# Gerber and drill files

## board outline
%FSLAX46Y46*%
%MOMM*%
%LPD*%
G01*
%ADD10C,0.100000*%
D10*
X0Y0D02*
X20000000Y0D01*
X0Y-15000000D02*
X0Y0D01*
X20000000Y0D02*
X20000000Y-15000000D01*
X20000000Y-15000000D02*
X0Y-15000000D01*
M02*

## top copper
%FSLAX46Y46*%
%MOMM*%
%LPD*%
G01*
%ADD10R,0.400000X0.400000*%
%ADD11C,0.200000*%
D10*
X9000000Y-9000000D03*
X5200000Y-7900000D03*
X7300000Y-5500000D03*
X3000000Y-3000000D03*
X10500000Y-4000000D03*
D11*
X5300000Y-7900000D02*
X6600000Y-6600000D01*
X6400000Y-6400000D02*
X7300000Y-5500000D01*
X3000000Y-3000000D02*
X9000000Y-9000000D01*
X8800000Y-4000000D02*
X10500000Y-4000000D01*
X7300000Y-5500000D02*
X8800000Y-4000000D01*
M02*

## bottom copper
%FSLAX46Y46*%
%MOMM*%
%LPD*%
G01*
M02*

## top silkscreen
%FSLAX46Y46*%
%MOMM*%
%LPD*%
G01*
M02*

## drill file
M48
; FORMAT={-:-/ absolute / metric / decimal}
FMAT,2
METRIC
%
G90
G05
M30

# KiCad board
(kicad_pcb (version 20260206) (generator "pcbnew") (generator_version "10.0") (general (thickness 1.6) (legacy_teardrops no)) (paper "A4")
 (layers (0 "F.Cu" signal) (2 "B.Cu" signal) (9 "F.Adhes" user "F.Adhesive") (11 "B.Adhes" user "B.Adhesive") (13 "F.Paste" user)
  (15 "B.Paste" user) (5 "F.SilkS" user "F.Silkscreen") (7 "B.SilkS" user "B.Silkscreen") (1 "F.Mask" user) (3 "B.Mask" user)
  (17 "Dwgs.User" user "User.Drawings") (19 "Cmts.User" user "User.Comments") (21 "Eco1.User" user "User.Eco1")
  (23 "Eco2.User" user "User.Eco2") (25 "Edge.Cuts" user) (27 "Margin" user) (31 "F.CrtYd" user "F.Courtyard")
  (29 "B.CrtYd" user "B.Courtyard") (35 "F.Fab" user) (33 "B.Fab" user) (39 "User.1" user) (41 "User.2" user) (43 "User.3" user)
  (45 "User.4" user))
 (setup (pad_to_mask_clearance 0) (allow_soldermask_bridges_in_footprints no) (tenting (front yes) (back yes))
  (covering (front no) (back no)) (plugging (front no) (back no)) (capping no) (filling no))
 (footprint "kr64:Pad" (layer "F.Cu") (at 9 9)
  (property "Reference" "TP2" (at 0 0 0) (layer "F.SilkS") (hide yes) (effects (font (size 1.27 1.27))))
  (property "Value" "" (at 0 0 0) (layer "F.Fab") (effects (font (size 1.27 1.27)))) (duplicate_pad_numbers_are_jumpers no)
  (pad "1" smd rect (at 0 0) (size 0.4 0.4) (layers "F.Cu" "F.Mask" "F.Paste") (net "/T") (thermal_bridge_angle 45)))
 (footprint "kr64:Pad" (layer "F.Cu") (at 5.2 7.9)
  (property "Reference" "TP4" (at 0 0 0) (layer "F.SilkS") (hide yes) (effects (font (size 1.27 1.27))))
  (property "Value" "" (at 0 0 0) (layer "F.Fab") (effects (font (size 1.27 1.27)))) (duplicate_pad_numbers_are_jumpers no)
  (pad "1" smd rect (at 0 0) (size 0.4 0.4) (layers "F.Cu" "F.Mask" "F.Paste") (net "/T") (thermal_bridge_angle 45)))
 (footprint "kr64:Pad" (layer "F.Cu") (at 7.3 5.5)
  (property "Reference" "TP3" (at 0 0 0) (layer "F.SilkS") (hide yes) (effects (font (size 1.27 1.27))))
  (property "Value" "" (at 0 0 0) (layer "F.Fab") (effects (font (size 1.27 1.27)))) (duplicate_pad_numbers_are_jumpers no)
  (pad "1" smd rect (at 0 0) (size 0.4 0.4) (layers "F.Cu" "F.Mask" "F.Paste") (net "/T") (thermal_bridge_angle 45)))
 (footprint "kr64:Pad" (layer "F.Cu") (at 3 3)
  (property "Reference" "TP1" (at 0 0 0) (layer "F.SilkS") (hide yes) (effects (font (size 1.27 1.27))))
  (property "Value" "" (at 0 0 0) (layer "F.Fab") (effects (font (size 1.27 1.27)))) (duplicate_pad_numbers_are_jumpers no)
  (pad "1" smd rect (at 0 0) (size 0.4 0.4) (layers "F.Cu" "F.Mask" "F.Paste") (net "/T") (thermal_bridge_angle 45)))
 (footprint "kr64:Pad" (layer "F.Cu") (at 10.5 4)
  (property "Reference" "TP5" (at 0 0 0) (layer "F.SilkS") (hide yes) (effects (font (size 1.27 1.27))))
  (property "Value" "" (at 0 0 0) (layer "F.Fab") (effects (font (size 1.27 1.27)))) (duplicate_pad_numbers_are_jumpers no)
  (pad "1" smd rect (at 0 0) (size 0.4 0.4) (layers "F.Cu" "F.Mask" "F.Paste") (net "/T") (thermal_bridge_angle 45)))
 (gr_line (start 0 0) (end 20 0) (stroke (width 0.1) (type default)) (layer "Edge.Cuts"))
 (gr_line (start 0 15) (end 0 0) (stroke (width 0.1) (type default)) (layer "Edge.Cuts"))
 (gr_line (start 20 0) (end 20 15) (stroke (width 0.1) (type default)) (layer "Edge.Cuts"))
 (gr_line (start 20 15) (end 0 15) (stroke (width 0.1) (type default)) (layer "Edge.Cuts"))
 (segment (start 5.3 7.9) (end 6.6 6.6) (width 0.2) (layer "F.Cu") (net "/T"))
 (segment (start 6.4 6.4) (end 7.3 5.5) (width 0.2) (layer "F.Cu") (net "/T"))
 (segment (start 3 3) (end 9 9) (width 0.2) (layer "F.Cu") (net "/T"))
 (segment (start 8.8 4) (end 10.5 4) (width 0.2) (layer "F.Cu") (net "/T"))
 (segment (start 7.3 5.5) (end 8.8 4) (width 0.2) (layer "F.Cu") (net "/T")))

